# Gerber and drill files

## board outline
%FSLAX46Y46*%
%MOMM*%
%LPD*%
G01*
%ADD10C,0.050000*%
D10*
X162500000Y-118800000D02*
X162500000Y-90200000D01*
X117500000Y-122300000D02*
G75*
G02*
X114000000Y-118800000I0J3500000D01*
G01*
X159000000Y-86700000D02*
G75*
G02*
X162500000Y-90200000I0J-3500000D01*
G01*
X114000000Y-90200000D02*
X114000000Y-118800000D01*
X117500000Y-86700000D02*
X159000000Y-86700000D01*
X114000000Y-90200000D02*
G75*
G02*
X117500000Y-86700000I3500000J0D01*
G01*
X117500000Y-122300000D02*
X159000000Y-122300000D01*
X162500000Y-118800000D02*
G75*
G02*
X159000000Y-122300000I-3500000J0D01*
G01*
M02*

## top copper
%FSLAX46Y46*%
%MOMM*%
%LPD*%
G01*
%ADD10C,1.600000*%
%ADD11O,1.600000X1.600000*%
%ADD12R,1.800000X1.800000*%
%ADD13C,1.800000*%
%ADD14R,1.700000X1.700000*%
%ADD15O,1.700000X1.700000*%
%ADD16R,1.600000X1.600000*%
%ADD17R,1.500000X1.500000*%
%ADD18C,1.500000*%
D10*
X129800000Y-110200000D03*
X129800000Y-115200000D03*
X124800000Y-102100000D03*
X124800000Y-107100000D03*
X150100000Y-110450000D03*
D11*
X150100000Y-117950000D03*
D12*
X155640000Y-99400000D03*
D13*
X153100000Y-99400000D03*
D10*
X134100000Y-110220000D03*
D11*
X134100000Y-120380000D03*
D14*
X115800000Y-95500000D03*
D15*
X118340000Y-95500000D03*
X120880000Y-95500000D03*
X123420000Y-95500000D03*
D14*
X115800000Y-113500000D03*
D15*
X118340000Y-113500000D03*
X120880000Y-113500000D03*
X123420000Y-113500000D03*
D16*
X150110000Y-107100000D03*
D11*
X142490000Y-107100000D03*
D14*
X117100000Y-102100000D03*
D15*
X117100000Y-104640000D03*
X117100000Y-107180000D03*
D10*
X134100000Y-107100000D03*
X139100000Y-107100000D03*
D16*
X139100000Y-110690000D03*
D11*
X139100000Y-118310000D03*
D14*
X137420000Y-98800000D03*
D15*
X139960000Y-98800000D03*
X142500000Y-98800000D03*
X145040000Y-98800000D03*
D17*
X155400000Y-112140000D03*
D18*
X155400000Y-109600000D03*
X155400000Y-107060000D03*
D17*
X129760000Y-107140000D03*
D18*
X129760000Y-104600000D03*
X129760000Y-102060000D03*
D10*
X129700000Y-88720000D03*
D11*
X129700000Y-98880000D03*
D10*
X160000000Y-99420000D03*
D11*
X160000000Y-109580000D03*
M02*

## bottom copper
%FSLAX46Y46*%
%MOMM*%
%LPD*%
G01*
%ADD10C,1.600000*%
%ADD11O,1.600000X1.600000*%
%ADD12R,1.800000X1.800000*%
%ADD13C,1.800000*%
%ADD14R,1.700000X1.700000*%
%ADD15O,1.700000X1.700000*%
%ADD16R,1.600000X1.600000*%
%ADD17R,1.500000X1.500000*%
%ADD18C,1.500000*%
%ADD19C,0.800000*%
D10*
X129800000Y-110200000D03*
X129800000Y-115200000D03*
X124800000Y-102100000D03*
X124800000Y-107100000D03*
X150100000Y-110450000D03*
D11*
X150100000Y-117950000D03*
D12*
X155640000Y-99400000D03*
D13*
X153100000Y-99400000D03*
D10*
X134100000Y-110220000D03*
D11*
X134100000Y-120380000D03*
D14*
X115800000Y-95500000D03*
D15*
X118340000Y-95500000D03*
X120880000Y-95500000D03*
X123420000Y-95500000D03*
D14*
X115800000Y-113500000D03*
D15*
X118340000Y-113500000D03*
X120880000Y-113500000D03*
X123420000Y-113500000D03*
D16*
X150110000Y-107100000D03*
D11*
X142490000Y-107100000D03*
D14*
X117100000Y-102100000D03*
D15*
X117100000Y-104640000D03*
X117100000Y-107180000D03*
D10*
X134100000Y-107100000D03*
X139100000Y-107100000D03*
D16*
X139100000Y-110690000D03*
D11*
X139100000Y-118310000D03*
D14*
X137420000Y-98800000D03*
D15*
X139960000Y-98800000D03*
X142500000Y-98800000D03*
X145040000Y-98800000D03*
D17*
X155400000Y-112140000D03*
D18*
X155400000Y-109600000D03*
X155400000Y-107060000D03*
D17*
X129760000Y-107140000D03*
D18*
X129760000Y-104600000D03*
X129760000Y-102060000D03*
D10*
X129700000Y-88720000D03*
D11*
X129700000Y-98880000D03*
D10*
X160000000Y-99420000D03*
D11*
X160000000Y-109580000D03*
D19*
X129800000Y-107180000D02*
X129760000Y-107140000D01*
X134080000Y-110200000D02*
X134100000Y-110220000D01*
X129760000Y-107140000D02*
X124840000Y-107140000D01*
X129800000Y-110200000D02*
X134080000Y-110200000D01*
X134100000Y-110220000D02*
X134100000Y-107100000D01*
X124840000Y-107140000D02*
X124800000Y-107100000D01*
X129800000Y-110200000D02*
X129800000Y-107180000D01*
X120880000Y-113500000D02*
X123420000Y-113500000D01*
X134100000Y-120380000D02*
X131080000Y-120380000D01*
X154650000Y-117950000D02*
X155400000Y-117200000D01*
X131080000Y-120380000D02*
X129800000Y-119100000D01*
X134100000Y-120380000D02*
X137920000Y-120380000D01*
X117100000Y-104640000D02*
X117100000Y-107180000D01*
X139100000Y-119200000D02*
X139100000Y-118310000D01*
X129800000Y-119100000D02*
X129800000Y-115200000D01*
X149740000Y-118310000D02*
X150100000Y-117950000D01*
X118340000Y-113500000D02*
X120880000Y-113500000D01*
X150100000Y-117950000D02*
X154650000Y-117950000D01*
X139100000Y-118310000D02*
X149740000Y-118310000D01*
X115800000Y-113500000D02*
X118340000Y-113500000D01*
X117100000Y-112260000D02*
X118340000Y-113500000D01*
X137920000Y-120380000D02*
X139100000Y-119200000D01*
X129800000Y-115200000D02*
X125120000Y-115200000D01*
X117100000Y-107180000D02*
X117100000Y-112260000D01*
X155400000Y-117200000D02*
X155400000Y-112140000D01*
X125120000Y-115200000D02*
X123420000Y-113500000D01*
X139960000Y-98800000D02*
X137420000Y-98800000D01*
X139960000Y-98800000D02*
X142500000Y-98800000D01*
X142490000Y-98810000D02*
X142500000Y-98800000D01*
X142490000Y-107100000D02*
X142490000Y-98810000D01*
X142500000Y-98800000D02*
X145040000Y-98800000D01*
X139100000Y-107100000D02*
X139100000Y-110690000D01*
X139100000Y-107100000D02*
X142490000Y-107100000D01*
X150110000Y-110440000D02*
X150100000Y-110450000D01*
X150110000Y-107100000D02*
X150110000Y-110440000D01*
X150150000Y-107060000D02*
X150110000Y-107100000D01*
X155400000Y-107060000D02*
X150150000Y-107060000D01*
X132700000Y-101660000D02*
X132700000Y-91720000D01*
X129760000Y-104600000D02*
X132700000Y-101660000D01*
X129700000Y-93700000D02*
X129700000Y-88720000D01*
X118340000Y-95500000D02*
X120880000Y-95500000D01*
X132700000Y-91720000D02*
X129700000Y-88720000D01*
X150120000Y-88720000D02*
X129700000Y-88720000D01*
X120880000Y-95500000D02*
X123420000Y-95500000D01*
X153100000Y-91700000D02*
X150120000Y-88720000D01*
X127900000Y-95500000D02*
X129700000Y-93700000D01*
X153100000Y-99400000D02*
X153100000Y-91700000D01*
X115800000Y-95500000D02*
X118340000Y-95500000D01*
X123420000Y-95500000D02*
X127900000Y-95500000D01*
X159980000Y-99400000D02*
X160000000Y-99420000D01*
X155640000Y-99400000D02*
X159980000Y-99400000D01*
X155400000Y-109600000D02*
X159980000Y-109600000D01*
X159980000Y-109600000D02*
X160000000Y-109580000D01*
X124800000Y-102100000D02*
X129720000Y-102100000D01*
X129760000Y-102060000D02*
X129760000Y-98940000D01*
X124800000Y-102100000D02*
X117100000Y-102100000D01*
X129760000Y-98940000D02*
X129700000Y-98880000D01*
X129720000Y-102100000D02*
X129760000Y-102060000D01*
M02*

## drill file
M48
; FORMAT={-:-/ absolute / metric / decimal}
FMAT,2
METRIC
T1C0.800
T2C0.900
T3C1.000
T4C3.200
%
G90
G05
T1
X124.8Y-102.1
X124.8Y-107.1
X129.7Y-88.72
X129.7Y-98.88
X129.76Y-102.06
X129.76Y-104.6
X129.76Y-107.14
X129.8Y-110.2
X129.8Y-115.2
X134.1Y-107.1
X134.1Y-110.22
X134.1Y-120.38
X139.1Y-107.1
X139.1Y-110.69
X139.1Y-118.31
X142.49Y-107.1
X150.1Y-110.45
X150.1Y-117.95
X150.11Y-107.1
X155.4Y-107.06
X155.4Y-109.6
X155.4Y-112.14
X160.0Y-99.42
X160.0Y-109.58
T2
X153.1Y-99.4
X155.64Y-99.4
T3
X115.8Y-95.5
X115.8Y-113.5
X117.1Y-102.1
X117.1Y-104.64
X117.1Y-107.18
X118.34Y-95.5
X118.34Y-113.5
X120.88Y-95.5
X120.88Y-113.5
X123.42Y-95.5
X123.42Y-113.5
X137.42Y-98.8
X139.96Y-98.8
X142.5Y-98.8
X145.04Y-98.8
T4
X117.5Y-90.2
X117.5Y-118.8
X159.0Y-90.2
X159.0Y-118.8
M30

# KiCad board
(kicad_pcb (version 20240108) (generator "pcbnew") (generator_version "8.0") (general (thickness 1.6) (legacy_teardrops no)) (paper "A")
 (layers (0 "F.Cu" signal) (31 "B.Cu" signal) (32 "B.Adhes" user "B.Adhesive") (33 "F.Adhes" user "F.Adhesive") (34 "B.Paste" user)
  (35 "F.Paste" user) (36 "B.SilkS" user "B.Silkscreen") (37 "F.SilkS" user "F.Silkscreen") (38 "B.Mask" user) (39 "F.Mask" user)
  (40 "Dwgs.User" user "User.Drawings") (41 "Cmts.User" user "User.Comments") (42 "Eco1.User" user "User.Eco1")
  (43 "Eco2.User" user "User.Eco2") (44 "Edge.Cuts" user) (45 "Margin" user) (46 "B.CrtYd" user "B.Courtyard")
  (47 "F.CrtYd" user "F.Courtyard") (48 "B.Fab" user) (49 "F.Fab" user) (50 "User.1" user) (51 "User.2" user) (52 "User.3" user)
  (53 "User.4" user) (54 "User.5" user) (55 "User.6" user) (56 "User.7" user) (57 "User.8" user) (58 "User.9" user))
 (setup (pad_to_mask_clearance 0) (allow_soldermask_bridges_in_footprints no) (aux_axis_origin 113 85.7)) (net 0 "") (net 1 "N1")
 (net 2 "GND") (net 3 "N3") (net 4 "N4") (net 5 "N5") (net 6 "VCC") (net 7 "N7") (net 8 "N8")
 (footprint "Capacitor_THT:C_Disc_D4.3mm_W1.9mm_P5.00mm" (layer "F.Cu") (at 129.8 110.2 -90)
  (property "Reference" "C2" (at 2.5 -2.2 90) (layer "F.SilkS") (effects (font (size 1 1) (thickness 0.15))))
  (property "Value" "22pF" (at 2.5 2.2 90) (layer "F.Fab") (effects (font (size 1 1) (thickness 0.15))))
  (pad "1" thru_hole circle (at 0 0 270) (size 1.6 1.6) (drill 0.8) (layers "*.Cu" "*.Mask") (remove_unused_layers no) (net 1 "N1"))
  (pad "2" thru_hole circle (at 5 0 270) (size 1.6 1.6) (drill 0.8) (layers "*.Cu" "*.Mask") (remove_unused_layers no) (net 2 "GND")))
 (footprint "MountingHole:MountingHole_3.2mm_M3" (layer "F.Cu") (at 117.5 90.2)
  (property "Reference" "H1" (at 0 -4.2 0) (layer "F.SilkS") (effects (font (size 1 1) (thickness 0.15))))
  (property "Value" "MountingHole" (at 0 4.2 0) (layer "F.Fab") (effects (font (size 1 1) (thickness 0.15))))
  (pad "" np_thru_hole circle (at 0 0) (size 3.2 3.2) (drill 3.2) (layers "*.Cu" "*.Mask")))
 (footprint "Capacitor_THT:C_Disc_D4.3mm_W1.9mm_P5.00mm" (layer "F.Cu") (at 124.8 102.1 -90)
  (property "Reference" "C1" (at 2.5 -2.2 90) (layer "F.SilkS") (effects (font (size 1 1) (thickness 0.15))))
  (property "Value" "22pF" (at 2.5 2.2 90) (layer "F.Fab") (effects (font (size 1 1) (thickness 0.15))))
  (pad "1" thru_hole circle (at 0 0 270) (size 1.6 1.6) (drill 0.8) (layers "*.Cu" "*.Mask") (remove_unused_layers no) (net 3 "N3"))
  (pad "2" thru_hole circle (at 5 0 270) (size 1.6 1.6) (drill 0.8) (layers "*.Cu" "*.Mask") (remove_unused_layers no) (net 1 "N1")))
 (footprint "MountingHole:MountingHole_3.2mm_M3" (layer "F.Cu") (at 159 118.8)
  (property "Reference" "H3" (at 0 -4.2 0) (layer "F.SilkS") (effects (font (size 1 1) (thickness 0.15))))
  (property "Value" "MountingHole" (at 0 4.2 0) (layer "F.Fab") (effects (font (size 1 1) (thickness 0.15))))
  (pad "" np_thru_hole circle (at 0 0) (size 3.2 3.2) (drill 3.2) (layers "*.Cu" "*.Mask")))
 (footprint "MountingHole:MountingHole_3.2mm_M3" (layer "F.Cu") (at 159 90.2)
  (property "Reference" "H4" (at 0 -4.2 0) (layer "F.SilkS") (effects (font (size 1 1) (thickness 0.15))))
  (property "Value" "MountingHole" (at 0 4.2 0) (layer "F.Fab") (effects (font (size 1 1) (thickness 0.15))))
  (pad "" np_thru_hole circle (at 0 0) (size 3.2 3.2) (drill 3.2) (layers "*.Cu" "*.Mask")))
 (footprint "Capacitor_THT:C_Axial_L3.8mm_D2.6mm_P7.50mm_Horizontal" (layer "F.Cu") (at 150.1 110.45 -90)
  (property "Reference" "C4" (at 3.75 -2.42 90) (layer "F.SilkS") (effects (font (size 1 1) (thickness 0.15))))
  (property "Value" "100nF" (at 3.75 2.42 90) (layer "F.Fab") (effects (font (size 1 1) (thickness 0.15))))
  (pad "1" thru_hole circle (at 0 0 270) (size 1.6 1.6) (drill 0.8) (layers "*.Cu" "*.Mask") (remove_unused_layers no) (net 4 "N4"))
  (pad "2" thru_hole oval (at 7.5 0 270) (size 1.6 1.6) (drill 0.8) (layers "*.Cu" "*.Mask") (remove_unused_layers no) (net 2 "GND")))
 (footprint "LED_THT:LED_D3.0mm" (layer "F.Cu") (at 155.64 99.4 180)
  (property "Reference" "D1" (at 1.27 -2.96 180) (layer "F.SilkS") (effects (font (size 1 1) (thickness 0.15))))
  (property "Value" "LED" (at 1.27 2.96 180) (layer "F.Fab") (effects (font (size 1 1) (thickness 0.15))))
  (pad "1" thru_hole rect (at 0 0 180) (size 1.8 1.8) (drill 0.9) (layers "*.Cu" "*.Mask") (remove_unused_layers no) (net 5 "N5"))
  (pad "2" thru_hole circle (at 2.54 0 180) (size 1.8 1.8) (drill 0.9) (layers "*.Cu" "*.Mask") (remove_unused_layers no) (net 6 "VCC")))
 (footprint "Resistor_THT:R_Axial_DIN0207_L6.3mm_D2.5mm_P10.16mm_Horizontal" (layer "F.Cu") (at 134.1 110.22 -90)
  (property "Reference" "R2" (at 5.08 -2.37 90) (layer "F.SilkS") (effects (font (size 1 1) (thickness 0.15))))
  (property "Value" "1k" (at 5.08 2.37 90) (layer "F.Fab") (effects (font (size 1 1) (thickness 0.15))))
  (pad "1" thru_hole circle (at 0 0 270) (size 1.6 1.6) (drill 0.8) (layers "*.Cu" "*.Mask") (remove_unused_layers no) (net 1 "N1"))
  (pad "2" thru_hole oval (at 10.16 0 270) (size 1.6 1.6) (drill 0.8) (layers "*.Cu" "*.Mask") (remove_unused_layers no) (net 2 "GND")))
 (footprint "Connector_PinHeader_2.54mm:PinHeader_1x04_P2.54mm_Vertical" (layer "F.Cu") (at 115.8 95.5 90)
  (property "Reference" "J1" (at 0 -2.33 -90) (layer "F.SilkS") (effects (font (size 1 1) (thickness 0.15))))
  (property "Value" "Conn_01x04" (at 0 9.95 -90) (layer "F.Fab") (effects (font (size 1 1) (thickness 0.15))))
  (pad "1" thru_hole rect (at 0 0 90) (size 1.7 1.7) (drill 1) (layers "*.Cu" "*.Mask") (remove_unused_layers no) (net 6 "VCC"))
  (pad "2" thru_hole oval (at 0 2.54 90) (size 1.7 1.7) (drill 1) (layers "*.Cu" "*.Mask") (remove_unused_layers no) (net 6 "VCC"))
  (pad "3" thru_hole oval (at 0 5.08 90) (size 1.7 1.7) (drill 1) (layers "*.Cu" "*.Mask") (remove_unused_layers no) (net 6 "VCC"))
  (pad "4" thru_hole oval (at 0 7.62 90) (size 1.7 1.7) (drill 1) (layers "*.Cu" "*.Mask") (remove_unused_layers no) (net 6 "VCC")))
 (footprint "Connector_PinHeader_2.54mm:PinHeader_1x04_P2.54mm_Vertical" (layer "F.Cu") (at 115.8 113.5 90)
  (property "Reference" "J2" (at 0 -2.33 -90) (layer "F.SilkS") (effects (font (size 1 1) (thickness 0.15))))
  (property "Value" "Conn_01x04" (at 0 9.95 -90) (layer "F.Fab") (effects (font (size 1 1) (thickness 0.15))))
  (pad "1" thru_hole rect (at 0 0 90) (size 1.7 1.7) (drill 1) (layers "*.Cu" "*.Mask") (remove_unused_layers no) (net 2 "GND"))
  (pad "2" thru_hole oval (at 0 2.54 90) (size 1.7 1.7) (drill 1) (layers "*.Cu" "*.Mask") (remove_unused_layers no) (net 2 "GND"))
  (pad "3" thru_hole oval (at 0 5.08 90) (size 1.7 1.7) (drill 1) (layers "*.Cu" "*.Mask") (remove_unused_layers no) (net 2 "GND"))
  (pad "4" thru_hole oval (at 0 7.62 90) (size 1.7 1.7) (drill 1) (layers "*.Cu" "*.Mask") (remove_unused_layers no) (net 2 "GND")))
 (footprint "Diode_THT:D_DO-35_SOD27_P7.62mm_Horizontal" (layer "F.Cu") (at 150.11 107.1 180)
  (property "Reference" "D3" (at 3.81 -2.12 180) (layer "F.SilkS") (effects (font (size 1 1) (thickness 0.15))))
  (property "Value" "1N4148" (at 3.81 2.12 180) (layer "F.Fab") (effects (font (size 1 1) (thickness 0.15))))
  (pad "1" thru_hole rect (at 0 0 180) (size 1.6 1.6) (drill 0.8) (layers "*.Cu" "*.Mask") (remove_unused_layers no) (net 4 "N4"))
  (pad "2" thru_hole oval (at 7.62 0 180) (size 1.6 1.6) (drill 0.8) (layers "*.Cu" "*.Mask") (remove_unused_layers no) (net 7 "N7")))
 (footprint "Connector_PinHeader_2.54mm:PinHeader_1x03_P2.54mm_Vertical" (layer "F.Cu") (at 117.1 102.1)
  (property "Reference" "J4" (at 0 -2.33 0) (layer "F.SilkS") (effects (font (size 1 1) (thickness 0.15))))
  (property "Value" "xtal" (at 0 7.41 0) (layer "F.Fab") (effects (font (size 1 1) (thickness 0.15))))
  (pad "1" thru_hole rect (at 0 0) (size 1.7 1.7) (drill 1) (layers "*.Cu" "*.Mask") (remove_unused_layers no) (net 3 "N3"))
  (pad "2" thru_hole oval (at 0 2.54) (size 1.7 1.7) (drill 1) (layers "*.Cu" "*.Mask") (remove_unused_layers no) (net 2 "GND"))
  (pad "3" thru_hole oval (at 0 5.08) (size 1.7 1.7) (drill 1) (layers "*.Cu" "*.Mask") (remove_unused_layers no) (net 2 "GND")))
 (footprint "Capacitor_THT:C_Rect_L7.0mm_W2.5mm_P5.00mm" (layer "F.Cu") (at 134.1 107.1)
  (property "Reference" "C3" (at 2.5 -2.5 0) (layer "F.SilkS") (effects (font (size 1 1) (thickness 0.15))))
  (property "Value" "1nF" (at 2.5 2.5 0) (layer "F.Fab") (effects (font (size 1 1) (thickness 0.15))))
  (pad "1" thru_hole circle (at 0 0) (size 1.6 1.6) (drill 0.8) (layers "*.Cu" "*.Mask") (remove_unused_layers no) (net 1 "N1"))
  (pad "2" thru_hole circle (at 5 0) (size 1.6 1.6) (drill 0.8) (layers "*.Cu" "*.Mask") (remove_unused_layers no) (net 7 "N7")))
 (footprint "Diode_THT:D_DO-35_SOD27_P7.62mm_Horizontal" (layer "F.Cu") (at 139.1 110.69 -90)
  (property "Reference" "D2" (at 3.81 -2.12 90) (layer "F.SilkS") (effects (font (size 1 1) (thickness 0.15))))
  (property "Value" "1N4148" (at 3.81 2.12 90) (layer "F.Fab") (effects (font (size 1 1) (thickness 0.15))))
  (pad "1" thru_hole rect (at 0 0 270) (size 1.6 1.6) (drill 0.8) (layers "*.Cu" "*.Mask") (remove_unused_layers no) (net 7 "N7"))
  (pad "2" thru_hole oval (at 7.62 0 270) (size 1.6 1.6) (drill 0.8) (layers "*.Cu" "*.Mask") (remove_unused_layers no) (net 2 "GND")))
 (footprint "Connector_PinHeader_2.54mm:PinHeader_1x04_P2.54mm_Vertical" (layer "F.Cu") (at 137.42 98.8 90)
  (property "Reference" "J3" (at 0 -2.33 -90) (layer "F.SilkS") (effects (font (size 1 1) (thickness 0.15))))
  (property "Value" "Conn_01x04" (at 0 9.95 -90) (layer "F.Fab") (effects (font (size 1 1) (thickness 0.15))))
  (pad "1" thru_hole rect (at 0 0 90) (size 1.7 1.7) (drill 1) (layers "*.Cu" "*.Mask") (remove_unused_layers no) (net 7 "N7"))
  (pad "2" thru_hole oval (at 0 2.54 90) (size 1.7 1.7) (drill 1) (layers "*.Cu" "*.Mask") (remove_unused_layers no) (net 7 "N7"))
  (pad "3" thru_hole oval (at 0 5.08 90) (size 1.7 1.7) (drill 1) (layers "*.Cu" "*.Mask") (remove_unused_layers no) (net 7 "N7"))
  (pad "4" thru_hole oval (at 0 7.62 90) (size 1.7 1.7) (drill 1) (layers "*.Cu" "*.Mask") (remove_unused_layers no) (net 7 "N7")))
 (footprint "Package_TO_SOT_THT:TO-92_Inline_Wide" (layer "F.Cu") (at 155.4 112.14 90)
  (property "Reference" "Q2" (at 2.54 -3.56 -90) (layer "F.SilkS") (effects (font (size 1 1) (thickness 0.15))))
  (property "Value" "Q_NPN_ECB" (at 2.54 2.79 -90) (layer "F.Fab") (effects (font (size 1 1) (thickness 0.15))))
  (pad "1" thru_hole rect (at 0 0 90) (size 1.5 1.5) (drill 0.8) (layers "*.Cu" "*.Mask") (remove_unused_layers no) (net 2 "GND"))
  (pad "2" thru_hole circle (at 2.54 0 90) (size 1.5 1.5) (drill 0.8) (layers "*.Cu" "*.Mask") (remove_unused_layers no) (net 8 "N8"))
  (pad "3" thru_hole circle (at 5.08 0 90) (size 1.5 1.5) (drill 0.8) (layers "*.Cu" "*.Mask") (remove_unused_layers no) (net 4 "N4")))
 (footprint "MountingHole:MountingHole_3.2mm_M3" (layer "F.Cu") (at 117.5 118.8)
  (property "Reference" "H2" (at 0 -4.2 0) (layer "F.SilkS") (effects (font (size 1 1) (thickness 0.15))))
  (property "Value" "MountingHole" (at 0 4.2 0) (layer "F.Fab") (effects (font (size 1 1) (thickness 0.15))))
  (pad "" np_thru_hole circle (at 0 0) (size 3.2 3.2) (drill 3.2) (layers "*.Cu" "*.Mask")))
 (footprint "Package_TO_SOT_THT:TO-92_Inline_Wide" (layer "F.Cu") (at 129.76 107.14 90)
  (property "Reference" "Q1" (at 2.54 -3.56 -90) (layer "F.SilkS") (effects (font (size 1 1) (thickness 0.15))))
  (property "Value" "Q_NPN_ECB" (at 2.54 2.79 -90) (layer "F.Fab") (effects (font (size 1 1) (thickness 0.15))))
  (pad "1" thru_hole rect (at 0 0 90) (size 1.5 1.5) (drill 0.8) (layers "*.Cu" "*.Mask") (remove_unused_layers no) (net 1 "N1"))
  (pad "2" thru_hole circle (at 2.54 0 90) (size 1.5 1.5) (drill 0.8) (layers "*.Cu" "*.Mask") (remove_unused_layers no) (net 6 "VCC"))
  (pad "3" thru_hole circle (at 5.08 0 90) (size 1.5 1.5) (drill 0.8) (layers "*.Cu" "*.Mask") (remove_unused_layers no) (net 3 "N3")))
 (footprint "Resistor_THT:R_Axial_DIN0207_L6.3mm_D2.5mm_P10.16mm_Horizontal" (layer "F.Cu") (at 129.7 88.72 -90)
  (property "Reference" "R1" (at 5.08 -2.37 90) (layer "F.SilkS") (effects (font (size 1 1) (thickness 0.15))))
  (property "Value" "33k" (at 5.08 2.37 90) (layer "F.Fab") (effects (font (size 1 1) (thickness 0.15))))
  (pad "1" thru_hole circle (at 0 0 270) (size 1.6 1.6) (drill 0.8) (layers "*.Cu" "*.Mask") (remove_unused_layers no) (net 6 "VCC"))
  (pad "2" thru_hole oval (at 10.16 0 270) (size 1.6 1.6) (drill 0.8) (layers "*.Cu" "*.Mask") (remove_unused_layers no) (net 3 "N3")))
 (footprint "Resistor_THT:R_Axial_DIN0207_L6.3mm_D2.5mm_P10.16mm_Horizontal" (layer "F.Cu") (at 160 99.42 -90)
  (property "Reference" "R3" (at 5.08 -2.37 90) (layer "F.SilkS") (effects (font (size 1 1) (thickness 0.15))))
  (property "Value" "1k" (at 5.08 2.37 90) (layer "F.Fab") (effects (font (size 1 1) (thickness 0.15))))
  (pad "1" thru_hole circle (at 0 0 270) (size 1.6 1.6) (drill 0.8) (layers "*.Cu" "*.Mask") (remove_unused_layers no) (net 5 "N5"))
  (pad "2" thru_hole oval (at 10.16 0 270) (size 1.6 1.6) (drill 0.8) (layers "*.Cu" "*.Mask") (remove_unused_layers no) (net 8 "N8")))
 (gr_line (start 162.5 118.8) (end 162.5 90.2) (stroke (width 0.05) (type default)) (layer "Edge.Cuts"))
 (gr_arc (start 117.5 122.3) (mid 115.025126 121.274874) (end 114 118.8) (stroke (width 0.05) (type default)) (layer "Edge.Cuts"))
 (gr_arc (start 159 86.7) (mid 161.474874 87.725126) (end 162.5 90.2) (stroke (width 0.05) (type default)) (layer "Edge.Cuts"))
 (gr_line (start 114 90.2) (end 114 118.8) (stroke (width 0.05) (type default)) (layer "Edge.Cuts"))
 (gr_line (start 117.5 86.7) (end 159 86.7) (stroke (width 0.05) (type default)) (layer "Edge.Cuts"))
 (gr_arc (start 114 90.2) (mid 115.025126 87.725126) (end 117.5 86.7) (stroke (width 0.05) (type default)) (layer "Edge.Cuts"))
 (gr_line (start 117.5 122.3) (end 159 122.3) (stroke (width 0.05) (type default)) (layer "Edge.Cuts"))
 (gr_arc (start 162.5 118.8) (mid 161.474874 121.274874) (end 159 122.3) (stroke (width 0.05) (type default)) (layer "Edge.Cuts"))
 (segment (start 129.8 107.18) (end 129.76 107.14) (width 0.8) (layer "B.Cu") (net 1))
 (segment (start 134.08 110.2) (end 134.1 110.22) (width 0.8) (layer "B.Cu") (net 1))
 (segment (start 129.76 107.14) (end 124.84 107.14) (width 0.8) (layer "B.Cu") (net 1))
 (segment (start 129.8 110.2) (end 134.08 110.2) (width 0.8) (layer "B.Cu") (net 1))
 (segment (start 134.1 110.22) (end 134.1 107.1) (width 0.8) (layer "B.Cu") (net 1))
 (segment (start 124.84 107.14) (end 124.8 107.1) (width 0.8) (layer "B.Cu") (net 1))
 (segment (start 129.8 110.2) (end 129.8 107.18) (width 0.8) (layer "B.Cu") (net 1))
 (segment (start 120.88 113.5) (end 123.42 113.5) (width 0.8) (layer "B.Cu") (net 2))
 (segment (start 134.1 120.38) (end 131.08 120.38) (width 0.8) (layer "B.Cu") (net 2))
 (segment (start 154.65 117.95) (end 155.4 117.2) (width 0.8) (layer "B.Cu") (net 2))
 (segment (start 131.08 120.38) (end 129.8 119.1) (width 0.8) (layer "B.Cu") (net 2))
 (segment (start 134.1 120.38) (end 137.92 120.38) (width 0.8) (layer "B.Cu") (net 2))
 (segment (start 117.1 104.64) (end 117.1 107.18) (width 0.8) (layer "B.Cu") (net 2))
 (segment (start 139.1 119.2) (end 139.1 118.31) (width 0.8) (layer "B.Cu") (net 2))
 (segment (start 129.8 119.1) (end 129.8 115.2) (width 0.8) (layer "B.Cu") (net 2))
 (segment (start 149.74 118.31) (end 150.1 117.95) (width 0.8) (layer "B.Cu") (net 2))
 (segment (start 118.34 113.5) (end 120.88 113.5) (width 0.8) (layer "B.Cu") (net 2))
 (segment (start 150.1 117.95) (end 154.65 117.95) (width 0.8) (layer "B.Cu") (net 2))
 (segment (start 139.1 118.31) (end 149.74 118.31) (width 0.8) (layer "B.Cu") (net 2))
 (segment (start 115.8 113.5) (end 118.34 113.5) (width 0.8) (layer "B.Cu") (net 2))
 (segment (start 117.1 112.26) (end 118.34 113.5) (width 0.8) (layer "B.Cu") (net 2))
 (segment (start 137.92 120.38) (end 139.1 119.2) (width 0.8) (layer "B.Cu") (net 2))
 (segment (start 129.8 115.2) (end 125.12 115.2) (width 0.8) (layer "B.Cu") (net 2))
 (segment (start 117.1 107.18) (end 117.1 112.26) (width 0.8) (layer "B.Cu") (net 2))
 (segment (start 155.4 117.2) (end 155.4 112.14) (width 0.8) (layer "B.Cu") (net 2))
 (segment (start 125.12 115.2) (end 123.42 113.5) (width 0.8) (layer "B.Cu") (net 2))
 (segment (start 139.96 98.8) (end 137.42 98.8) (width 0.8) (layer "B.Cu") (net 7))
 (segment (start 139.96 98.8) (end 142.5 98.8) (width 0.8) (layer "B.Cu") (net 7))
 (segment (start 142.49 98.81) (end 142.5 98.8) (width 0.8) (layer "B.Cu") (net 7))
 (segment (start 142.49 107.1) (end 142.49 98.81) (width 0.8) (layer "B.Cu") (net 7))
 (segment (start 142.5 98.8) (end 145.04 98.8) (width 0.8) (layer "B.Cu") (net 7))
 (segment (start 139.1 107.1) (end 139.1 110.69) (width 0.8) (layer "B.Cu") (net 7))
 (segment (start 139.1 107.1) (end 142.49 107.1) (width 0.8) (layer "B.Cu") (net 7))
 (segment (start 150.11 110.44) (end 150.1 110.45) (width 0.8) (layer "B.Cu") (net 4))
 (segment (start 150.11 107.1) (end 150.11 110.44) (width 0.8) (layer "B.Cu") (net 4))
 (segment (start 150.15 107.06) (end 150.11 107.1) (width 0.8) (layer "B.Cu") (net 4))
 (segment (start 155.4 107.06) (end 150.15 107.06) (width 0.8) (layer "B.Cu") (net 4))
 (segment (start 132.7 101.66) (end 132.7 91.72) (width 0.8) (layer "B.Cu") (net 6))
 (segment (start 129.76 104.6) (end 132.7 101.66) (width 0.8) (layer "B.Cu") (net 6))
 (segment (start 129.7 93.7) (end 129.7 88.72) (width 0.8) (layer "B.Cu") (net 6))
 (segment (start 118.34 95.5) (end 120.88 95.5) (width 0.8) (layer "B.Cu") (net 6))
 (segment (start 132.7 91.72) (end 129.7 88.72) (width 0.8) (layer "B.Cu") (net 6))
 (segment (start 150.12 88.72) (end 129.7 88.72) (width 0.8) (layer "B.Cu") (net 6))
 (segment (start 120.88 95.5) (end 123.42 95.5) (width 0.8) (layer "B.Cu") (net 6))
 (segment (start 153.1 91.7) (end 150.12 88.72) (width 0.8) (layer "B.Cu") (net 6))
 (segment (start 127.9 95.5) (end 129.7 93.7) (width 0.8) (layer "B.Cu") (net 6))
 (segment (start 153.1 99.4) (end 153.1 91.7) (width 0.8) (layer "B.Cu") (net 6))
 (segment (start 115.8 95.5) (end 118.34 95.5) (width 0.8) (layer "B.Cu") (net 6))
 (segment (start 123.42 95.5) (end 127.9 95.5) (width 0.8) (layer "B.Cu") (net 6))
 (segment (start 159.98 99.4) (end 160 99.42) (width 0.8) (layer "B.Cu") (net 5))
 (segment (start 155.64 99.4) (end 159.98 99.4) (width 0.8) (layer "B.Cu") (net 5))
 (segment (start 155.4 109.6) (end 159.98 109.6) (width 0.8) (layer "B.Cu") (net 8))
 (segment (start 159.98 109.6) (end 160 109.58) (width 0.8) (layer "B.Cu") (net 8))
 (segment (start 124.8 102.1) (end 129.72 102.1) (width 0.8) (layer "B.Cu") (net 3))
 (segment (start 129.76 102.06) (end 129.76 98.94) (width 0.8) (layer "B.Cu") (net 3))
 (segment (start 124.8 102.1) (end 117.1 102.1) (width 0.8) (layer "B.Cu") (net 3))
 (segment (start 129.76 98.94) (end 129.7 98.88) (width 0.8) (layer "B.Cu") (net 3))
 (segment (start 129.72 102.1) (end 129.76 102.06) (width 0.8) (layer "B.Cu") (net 3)))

